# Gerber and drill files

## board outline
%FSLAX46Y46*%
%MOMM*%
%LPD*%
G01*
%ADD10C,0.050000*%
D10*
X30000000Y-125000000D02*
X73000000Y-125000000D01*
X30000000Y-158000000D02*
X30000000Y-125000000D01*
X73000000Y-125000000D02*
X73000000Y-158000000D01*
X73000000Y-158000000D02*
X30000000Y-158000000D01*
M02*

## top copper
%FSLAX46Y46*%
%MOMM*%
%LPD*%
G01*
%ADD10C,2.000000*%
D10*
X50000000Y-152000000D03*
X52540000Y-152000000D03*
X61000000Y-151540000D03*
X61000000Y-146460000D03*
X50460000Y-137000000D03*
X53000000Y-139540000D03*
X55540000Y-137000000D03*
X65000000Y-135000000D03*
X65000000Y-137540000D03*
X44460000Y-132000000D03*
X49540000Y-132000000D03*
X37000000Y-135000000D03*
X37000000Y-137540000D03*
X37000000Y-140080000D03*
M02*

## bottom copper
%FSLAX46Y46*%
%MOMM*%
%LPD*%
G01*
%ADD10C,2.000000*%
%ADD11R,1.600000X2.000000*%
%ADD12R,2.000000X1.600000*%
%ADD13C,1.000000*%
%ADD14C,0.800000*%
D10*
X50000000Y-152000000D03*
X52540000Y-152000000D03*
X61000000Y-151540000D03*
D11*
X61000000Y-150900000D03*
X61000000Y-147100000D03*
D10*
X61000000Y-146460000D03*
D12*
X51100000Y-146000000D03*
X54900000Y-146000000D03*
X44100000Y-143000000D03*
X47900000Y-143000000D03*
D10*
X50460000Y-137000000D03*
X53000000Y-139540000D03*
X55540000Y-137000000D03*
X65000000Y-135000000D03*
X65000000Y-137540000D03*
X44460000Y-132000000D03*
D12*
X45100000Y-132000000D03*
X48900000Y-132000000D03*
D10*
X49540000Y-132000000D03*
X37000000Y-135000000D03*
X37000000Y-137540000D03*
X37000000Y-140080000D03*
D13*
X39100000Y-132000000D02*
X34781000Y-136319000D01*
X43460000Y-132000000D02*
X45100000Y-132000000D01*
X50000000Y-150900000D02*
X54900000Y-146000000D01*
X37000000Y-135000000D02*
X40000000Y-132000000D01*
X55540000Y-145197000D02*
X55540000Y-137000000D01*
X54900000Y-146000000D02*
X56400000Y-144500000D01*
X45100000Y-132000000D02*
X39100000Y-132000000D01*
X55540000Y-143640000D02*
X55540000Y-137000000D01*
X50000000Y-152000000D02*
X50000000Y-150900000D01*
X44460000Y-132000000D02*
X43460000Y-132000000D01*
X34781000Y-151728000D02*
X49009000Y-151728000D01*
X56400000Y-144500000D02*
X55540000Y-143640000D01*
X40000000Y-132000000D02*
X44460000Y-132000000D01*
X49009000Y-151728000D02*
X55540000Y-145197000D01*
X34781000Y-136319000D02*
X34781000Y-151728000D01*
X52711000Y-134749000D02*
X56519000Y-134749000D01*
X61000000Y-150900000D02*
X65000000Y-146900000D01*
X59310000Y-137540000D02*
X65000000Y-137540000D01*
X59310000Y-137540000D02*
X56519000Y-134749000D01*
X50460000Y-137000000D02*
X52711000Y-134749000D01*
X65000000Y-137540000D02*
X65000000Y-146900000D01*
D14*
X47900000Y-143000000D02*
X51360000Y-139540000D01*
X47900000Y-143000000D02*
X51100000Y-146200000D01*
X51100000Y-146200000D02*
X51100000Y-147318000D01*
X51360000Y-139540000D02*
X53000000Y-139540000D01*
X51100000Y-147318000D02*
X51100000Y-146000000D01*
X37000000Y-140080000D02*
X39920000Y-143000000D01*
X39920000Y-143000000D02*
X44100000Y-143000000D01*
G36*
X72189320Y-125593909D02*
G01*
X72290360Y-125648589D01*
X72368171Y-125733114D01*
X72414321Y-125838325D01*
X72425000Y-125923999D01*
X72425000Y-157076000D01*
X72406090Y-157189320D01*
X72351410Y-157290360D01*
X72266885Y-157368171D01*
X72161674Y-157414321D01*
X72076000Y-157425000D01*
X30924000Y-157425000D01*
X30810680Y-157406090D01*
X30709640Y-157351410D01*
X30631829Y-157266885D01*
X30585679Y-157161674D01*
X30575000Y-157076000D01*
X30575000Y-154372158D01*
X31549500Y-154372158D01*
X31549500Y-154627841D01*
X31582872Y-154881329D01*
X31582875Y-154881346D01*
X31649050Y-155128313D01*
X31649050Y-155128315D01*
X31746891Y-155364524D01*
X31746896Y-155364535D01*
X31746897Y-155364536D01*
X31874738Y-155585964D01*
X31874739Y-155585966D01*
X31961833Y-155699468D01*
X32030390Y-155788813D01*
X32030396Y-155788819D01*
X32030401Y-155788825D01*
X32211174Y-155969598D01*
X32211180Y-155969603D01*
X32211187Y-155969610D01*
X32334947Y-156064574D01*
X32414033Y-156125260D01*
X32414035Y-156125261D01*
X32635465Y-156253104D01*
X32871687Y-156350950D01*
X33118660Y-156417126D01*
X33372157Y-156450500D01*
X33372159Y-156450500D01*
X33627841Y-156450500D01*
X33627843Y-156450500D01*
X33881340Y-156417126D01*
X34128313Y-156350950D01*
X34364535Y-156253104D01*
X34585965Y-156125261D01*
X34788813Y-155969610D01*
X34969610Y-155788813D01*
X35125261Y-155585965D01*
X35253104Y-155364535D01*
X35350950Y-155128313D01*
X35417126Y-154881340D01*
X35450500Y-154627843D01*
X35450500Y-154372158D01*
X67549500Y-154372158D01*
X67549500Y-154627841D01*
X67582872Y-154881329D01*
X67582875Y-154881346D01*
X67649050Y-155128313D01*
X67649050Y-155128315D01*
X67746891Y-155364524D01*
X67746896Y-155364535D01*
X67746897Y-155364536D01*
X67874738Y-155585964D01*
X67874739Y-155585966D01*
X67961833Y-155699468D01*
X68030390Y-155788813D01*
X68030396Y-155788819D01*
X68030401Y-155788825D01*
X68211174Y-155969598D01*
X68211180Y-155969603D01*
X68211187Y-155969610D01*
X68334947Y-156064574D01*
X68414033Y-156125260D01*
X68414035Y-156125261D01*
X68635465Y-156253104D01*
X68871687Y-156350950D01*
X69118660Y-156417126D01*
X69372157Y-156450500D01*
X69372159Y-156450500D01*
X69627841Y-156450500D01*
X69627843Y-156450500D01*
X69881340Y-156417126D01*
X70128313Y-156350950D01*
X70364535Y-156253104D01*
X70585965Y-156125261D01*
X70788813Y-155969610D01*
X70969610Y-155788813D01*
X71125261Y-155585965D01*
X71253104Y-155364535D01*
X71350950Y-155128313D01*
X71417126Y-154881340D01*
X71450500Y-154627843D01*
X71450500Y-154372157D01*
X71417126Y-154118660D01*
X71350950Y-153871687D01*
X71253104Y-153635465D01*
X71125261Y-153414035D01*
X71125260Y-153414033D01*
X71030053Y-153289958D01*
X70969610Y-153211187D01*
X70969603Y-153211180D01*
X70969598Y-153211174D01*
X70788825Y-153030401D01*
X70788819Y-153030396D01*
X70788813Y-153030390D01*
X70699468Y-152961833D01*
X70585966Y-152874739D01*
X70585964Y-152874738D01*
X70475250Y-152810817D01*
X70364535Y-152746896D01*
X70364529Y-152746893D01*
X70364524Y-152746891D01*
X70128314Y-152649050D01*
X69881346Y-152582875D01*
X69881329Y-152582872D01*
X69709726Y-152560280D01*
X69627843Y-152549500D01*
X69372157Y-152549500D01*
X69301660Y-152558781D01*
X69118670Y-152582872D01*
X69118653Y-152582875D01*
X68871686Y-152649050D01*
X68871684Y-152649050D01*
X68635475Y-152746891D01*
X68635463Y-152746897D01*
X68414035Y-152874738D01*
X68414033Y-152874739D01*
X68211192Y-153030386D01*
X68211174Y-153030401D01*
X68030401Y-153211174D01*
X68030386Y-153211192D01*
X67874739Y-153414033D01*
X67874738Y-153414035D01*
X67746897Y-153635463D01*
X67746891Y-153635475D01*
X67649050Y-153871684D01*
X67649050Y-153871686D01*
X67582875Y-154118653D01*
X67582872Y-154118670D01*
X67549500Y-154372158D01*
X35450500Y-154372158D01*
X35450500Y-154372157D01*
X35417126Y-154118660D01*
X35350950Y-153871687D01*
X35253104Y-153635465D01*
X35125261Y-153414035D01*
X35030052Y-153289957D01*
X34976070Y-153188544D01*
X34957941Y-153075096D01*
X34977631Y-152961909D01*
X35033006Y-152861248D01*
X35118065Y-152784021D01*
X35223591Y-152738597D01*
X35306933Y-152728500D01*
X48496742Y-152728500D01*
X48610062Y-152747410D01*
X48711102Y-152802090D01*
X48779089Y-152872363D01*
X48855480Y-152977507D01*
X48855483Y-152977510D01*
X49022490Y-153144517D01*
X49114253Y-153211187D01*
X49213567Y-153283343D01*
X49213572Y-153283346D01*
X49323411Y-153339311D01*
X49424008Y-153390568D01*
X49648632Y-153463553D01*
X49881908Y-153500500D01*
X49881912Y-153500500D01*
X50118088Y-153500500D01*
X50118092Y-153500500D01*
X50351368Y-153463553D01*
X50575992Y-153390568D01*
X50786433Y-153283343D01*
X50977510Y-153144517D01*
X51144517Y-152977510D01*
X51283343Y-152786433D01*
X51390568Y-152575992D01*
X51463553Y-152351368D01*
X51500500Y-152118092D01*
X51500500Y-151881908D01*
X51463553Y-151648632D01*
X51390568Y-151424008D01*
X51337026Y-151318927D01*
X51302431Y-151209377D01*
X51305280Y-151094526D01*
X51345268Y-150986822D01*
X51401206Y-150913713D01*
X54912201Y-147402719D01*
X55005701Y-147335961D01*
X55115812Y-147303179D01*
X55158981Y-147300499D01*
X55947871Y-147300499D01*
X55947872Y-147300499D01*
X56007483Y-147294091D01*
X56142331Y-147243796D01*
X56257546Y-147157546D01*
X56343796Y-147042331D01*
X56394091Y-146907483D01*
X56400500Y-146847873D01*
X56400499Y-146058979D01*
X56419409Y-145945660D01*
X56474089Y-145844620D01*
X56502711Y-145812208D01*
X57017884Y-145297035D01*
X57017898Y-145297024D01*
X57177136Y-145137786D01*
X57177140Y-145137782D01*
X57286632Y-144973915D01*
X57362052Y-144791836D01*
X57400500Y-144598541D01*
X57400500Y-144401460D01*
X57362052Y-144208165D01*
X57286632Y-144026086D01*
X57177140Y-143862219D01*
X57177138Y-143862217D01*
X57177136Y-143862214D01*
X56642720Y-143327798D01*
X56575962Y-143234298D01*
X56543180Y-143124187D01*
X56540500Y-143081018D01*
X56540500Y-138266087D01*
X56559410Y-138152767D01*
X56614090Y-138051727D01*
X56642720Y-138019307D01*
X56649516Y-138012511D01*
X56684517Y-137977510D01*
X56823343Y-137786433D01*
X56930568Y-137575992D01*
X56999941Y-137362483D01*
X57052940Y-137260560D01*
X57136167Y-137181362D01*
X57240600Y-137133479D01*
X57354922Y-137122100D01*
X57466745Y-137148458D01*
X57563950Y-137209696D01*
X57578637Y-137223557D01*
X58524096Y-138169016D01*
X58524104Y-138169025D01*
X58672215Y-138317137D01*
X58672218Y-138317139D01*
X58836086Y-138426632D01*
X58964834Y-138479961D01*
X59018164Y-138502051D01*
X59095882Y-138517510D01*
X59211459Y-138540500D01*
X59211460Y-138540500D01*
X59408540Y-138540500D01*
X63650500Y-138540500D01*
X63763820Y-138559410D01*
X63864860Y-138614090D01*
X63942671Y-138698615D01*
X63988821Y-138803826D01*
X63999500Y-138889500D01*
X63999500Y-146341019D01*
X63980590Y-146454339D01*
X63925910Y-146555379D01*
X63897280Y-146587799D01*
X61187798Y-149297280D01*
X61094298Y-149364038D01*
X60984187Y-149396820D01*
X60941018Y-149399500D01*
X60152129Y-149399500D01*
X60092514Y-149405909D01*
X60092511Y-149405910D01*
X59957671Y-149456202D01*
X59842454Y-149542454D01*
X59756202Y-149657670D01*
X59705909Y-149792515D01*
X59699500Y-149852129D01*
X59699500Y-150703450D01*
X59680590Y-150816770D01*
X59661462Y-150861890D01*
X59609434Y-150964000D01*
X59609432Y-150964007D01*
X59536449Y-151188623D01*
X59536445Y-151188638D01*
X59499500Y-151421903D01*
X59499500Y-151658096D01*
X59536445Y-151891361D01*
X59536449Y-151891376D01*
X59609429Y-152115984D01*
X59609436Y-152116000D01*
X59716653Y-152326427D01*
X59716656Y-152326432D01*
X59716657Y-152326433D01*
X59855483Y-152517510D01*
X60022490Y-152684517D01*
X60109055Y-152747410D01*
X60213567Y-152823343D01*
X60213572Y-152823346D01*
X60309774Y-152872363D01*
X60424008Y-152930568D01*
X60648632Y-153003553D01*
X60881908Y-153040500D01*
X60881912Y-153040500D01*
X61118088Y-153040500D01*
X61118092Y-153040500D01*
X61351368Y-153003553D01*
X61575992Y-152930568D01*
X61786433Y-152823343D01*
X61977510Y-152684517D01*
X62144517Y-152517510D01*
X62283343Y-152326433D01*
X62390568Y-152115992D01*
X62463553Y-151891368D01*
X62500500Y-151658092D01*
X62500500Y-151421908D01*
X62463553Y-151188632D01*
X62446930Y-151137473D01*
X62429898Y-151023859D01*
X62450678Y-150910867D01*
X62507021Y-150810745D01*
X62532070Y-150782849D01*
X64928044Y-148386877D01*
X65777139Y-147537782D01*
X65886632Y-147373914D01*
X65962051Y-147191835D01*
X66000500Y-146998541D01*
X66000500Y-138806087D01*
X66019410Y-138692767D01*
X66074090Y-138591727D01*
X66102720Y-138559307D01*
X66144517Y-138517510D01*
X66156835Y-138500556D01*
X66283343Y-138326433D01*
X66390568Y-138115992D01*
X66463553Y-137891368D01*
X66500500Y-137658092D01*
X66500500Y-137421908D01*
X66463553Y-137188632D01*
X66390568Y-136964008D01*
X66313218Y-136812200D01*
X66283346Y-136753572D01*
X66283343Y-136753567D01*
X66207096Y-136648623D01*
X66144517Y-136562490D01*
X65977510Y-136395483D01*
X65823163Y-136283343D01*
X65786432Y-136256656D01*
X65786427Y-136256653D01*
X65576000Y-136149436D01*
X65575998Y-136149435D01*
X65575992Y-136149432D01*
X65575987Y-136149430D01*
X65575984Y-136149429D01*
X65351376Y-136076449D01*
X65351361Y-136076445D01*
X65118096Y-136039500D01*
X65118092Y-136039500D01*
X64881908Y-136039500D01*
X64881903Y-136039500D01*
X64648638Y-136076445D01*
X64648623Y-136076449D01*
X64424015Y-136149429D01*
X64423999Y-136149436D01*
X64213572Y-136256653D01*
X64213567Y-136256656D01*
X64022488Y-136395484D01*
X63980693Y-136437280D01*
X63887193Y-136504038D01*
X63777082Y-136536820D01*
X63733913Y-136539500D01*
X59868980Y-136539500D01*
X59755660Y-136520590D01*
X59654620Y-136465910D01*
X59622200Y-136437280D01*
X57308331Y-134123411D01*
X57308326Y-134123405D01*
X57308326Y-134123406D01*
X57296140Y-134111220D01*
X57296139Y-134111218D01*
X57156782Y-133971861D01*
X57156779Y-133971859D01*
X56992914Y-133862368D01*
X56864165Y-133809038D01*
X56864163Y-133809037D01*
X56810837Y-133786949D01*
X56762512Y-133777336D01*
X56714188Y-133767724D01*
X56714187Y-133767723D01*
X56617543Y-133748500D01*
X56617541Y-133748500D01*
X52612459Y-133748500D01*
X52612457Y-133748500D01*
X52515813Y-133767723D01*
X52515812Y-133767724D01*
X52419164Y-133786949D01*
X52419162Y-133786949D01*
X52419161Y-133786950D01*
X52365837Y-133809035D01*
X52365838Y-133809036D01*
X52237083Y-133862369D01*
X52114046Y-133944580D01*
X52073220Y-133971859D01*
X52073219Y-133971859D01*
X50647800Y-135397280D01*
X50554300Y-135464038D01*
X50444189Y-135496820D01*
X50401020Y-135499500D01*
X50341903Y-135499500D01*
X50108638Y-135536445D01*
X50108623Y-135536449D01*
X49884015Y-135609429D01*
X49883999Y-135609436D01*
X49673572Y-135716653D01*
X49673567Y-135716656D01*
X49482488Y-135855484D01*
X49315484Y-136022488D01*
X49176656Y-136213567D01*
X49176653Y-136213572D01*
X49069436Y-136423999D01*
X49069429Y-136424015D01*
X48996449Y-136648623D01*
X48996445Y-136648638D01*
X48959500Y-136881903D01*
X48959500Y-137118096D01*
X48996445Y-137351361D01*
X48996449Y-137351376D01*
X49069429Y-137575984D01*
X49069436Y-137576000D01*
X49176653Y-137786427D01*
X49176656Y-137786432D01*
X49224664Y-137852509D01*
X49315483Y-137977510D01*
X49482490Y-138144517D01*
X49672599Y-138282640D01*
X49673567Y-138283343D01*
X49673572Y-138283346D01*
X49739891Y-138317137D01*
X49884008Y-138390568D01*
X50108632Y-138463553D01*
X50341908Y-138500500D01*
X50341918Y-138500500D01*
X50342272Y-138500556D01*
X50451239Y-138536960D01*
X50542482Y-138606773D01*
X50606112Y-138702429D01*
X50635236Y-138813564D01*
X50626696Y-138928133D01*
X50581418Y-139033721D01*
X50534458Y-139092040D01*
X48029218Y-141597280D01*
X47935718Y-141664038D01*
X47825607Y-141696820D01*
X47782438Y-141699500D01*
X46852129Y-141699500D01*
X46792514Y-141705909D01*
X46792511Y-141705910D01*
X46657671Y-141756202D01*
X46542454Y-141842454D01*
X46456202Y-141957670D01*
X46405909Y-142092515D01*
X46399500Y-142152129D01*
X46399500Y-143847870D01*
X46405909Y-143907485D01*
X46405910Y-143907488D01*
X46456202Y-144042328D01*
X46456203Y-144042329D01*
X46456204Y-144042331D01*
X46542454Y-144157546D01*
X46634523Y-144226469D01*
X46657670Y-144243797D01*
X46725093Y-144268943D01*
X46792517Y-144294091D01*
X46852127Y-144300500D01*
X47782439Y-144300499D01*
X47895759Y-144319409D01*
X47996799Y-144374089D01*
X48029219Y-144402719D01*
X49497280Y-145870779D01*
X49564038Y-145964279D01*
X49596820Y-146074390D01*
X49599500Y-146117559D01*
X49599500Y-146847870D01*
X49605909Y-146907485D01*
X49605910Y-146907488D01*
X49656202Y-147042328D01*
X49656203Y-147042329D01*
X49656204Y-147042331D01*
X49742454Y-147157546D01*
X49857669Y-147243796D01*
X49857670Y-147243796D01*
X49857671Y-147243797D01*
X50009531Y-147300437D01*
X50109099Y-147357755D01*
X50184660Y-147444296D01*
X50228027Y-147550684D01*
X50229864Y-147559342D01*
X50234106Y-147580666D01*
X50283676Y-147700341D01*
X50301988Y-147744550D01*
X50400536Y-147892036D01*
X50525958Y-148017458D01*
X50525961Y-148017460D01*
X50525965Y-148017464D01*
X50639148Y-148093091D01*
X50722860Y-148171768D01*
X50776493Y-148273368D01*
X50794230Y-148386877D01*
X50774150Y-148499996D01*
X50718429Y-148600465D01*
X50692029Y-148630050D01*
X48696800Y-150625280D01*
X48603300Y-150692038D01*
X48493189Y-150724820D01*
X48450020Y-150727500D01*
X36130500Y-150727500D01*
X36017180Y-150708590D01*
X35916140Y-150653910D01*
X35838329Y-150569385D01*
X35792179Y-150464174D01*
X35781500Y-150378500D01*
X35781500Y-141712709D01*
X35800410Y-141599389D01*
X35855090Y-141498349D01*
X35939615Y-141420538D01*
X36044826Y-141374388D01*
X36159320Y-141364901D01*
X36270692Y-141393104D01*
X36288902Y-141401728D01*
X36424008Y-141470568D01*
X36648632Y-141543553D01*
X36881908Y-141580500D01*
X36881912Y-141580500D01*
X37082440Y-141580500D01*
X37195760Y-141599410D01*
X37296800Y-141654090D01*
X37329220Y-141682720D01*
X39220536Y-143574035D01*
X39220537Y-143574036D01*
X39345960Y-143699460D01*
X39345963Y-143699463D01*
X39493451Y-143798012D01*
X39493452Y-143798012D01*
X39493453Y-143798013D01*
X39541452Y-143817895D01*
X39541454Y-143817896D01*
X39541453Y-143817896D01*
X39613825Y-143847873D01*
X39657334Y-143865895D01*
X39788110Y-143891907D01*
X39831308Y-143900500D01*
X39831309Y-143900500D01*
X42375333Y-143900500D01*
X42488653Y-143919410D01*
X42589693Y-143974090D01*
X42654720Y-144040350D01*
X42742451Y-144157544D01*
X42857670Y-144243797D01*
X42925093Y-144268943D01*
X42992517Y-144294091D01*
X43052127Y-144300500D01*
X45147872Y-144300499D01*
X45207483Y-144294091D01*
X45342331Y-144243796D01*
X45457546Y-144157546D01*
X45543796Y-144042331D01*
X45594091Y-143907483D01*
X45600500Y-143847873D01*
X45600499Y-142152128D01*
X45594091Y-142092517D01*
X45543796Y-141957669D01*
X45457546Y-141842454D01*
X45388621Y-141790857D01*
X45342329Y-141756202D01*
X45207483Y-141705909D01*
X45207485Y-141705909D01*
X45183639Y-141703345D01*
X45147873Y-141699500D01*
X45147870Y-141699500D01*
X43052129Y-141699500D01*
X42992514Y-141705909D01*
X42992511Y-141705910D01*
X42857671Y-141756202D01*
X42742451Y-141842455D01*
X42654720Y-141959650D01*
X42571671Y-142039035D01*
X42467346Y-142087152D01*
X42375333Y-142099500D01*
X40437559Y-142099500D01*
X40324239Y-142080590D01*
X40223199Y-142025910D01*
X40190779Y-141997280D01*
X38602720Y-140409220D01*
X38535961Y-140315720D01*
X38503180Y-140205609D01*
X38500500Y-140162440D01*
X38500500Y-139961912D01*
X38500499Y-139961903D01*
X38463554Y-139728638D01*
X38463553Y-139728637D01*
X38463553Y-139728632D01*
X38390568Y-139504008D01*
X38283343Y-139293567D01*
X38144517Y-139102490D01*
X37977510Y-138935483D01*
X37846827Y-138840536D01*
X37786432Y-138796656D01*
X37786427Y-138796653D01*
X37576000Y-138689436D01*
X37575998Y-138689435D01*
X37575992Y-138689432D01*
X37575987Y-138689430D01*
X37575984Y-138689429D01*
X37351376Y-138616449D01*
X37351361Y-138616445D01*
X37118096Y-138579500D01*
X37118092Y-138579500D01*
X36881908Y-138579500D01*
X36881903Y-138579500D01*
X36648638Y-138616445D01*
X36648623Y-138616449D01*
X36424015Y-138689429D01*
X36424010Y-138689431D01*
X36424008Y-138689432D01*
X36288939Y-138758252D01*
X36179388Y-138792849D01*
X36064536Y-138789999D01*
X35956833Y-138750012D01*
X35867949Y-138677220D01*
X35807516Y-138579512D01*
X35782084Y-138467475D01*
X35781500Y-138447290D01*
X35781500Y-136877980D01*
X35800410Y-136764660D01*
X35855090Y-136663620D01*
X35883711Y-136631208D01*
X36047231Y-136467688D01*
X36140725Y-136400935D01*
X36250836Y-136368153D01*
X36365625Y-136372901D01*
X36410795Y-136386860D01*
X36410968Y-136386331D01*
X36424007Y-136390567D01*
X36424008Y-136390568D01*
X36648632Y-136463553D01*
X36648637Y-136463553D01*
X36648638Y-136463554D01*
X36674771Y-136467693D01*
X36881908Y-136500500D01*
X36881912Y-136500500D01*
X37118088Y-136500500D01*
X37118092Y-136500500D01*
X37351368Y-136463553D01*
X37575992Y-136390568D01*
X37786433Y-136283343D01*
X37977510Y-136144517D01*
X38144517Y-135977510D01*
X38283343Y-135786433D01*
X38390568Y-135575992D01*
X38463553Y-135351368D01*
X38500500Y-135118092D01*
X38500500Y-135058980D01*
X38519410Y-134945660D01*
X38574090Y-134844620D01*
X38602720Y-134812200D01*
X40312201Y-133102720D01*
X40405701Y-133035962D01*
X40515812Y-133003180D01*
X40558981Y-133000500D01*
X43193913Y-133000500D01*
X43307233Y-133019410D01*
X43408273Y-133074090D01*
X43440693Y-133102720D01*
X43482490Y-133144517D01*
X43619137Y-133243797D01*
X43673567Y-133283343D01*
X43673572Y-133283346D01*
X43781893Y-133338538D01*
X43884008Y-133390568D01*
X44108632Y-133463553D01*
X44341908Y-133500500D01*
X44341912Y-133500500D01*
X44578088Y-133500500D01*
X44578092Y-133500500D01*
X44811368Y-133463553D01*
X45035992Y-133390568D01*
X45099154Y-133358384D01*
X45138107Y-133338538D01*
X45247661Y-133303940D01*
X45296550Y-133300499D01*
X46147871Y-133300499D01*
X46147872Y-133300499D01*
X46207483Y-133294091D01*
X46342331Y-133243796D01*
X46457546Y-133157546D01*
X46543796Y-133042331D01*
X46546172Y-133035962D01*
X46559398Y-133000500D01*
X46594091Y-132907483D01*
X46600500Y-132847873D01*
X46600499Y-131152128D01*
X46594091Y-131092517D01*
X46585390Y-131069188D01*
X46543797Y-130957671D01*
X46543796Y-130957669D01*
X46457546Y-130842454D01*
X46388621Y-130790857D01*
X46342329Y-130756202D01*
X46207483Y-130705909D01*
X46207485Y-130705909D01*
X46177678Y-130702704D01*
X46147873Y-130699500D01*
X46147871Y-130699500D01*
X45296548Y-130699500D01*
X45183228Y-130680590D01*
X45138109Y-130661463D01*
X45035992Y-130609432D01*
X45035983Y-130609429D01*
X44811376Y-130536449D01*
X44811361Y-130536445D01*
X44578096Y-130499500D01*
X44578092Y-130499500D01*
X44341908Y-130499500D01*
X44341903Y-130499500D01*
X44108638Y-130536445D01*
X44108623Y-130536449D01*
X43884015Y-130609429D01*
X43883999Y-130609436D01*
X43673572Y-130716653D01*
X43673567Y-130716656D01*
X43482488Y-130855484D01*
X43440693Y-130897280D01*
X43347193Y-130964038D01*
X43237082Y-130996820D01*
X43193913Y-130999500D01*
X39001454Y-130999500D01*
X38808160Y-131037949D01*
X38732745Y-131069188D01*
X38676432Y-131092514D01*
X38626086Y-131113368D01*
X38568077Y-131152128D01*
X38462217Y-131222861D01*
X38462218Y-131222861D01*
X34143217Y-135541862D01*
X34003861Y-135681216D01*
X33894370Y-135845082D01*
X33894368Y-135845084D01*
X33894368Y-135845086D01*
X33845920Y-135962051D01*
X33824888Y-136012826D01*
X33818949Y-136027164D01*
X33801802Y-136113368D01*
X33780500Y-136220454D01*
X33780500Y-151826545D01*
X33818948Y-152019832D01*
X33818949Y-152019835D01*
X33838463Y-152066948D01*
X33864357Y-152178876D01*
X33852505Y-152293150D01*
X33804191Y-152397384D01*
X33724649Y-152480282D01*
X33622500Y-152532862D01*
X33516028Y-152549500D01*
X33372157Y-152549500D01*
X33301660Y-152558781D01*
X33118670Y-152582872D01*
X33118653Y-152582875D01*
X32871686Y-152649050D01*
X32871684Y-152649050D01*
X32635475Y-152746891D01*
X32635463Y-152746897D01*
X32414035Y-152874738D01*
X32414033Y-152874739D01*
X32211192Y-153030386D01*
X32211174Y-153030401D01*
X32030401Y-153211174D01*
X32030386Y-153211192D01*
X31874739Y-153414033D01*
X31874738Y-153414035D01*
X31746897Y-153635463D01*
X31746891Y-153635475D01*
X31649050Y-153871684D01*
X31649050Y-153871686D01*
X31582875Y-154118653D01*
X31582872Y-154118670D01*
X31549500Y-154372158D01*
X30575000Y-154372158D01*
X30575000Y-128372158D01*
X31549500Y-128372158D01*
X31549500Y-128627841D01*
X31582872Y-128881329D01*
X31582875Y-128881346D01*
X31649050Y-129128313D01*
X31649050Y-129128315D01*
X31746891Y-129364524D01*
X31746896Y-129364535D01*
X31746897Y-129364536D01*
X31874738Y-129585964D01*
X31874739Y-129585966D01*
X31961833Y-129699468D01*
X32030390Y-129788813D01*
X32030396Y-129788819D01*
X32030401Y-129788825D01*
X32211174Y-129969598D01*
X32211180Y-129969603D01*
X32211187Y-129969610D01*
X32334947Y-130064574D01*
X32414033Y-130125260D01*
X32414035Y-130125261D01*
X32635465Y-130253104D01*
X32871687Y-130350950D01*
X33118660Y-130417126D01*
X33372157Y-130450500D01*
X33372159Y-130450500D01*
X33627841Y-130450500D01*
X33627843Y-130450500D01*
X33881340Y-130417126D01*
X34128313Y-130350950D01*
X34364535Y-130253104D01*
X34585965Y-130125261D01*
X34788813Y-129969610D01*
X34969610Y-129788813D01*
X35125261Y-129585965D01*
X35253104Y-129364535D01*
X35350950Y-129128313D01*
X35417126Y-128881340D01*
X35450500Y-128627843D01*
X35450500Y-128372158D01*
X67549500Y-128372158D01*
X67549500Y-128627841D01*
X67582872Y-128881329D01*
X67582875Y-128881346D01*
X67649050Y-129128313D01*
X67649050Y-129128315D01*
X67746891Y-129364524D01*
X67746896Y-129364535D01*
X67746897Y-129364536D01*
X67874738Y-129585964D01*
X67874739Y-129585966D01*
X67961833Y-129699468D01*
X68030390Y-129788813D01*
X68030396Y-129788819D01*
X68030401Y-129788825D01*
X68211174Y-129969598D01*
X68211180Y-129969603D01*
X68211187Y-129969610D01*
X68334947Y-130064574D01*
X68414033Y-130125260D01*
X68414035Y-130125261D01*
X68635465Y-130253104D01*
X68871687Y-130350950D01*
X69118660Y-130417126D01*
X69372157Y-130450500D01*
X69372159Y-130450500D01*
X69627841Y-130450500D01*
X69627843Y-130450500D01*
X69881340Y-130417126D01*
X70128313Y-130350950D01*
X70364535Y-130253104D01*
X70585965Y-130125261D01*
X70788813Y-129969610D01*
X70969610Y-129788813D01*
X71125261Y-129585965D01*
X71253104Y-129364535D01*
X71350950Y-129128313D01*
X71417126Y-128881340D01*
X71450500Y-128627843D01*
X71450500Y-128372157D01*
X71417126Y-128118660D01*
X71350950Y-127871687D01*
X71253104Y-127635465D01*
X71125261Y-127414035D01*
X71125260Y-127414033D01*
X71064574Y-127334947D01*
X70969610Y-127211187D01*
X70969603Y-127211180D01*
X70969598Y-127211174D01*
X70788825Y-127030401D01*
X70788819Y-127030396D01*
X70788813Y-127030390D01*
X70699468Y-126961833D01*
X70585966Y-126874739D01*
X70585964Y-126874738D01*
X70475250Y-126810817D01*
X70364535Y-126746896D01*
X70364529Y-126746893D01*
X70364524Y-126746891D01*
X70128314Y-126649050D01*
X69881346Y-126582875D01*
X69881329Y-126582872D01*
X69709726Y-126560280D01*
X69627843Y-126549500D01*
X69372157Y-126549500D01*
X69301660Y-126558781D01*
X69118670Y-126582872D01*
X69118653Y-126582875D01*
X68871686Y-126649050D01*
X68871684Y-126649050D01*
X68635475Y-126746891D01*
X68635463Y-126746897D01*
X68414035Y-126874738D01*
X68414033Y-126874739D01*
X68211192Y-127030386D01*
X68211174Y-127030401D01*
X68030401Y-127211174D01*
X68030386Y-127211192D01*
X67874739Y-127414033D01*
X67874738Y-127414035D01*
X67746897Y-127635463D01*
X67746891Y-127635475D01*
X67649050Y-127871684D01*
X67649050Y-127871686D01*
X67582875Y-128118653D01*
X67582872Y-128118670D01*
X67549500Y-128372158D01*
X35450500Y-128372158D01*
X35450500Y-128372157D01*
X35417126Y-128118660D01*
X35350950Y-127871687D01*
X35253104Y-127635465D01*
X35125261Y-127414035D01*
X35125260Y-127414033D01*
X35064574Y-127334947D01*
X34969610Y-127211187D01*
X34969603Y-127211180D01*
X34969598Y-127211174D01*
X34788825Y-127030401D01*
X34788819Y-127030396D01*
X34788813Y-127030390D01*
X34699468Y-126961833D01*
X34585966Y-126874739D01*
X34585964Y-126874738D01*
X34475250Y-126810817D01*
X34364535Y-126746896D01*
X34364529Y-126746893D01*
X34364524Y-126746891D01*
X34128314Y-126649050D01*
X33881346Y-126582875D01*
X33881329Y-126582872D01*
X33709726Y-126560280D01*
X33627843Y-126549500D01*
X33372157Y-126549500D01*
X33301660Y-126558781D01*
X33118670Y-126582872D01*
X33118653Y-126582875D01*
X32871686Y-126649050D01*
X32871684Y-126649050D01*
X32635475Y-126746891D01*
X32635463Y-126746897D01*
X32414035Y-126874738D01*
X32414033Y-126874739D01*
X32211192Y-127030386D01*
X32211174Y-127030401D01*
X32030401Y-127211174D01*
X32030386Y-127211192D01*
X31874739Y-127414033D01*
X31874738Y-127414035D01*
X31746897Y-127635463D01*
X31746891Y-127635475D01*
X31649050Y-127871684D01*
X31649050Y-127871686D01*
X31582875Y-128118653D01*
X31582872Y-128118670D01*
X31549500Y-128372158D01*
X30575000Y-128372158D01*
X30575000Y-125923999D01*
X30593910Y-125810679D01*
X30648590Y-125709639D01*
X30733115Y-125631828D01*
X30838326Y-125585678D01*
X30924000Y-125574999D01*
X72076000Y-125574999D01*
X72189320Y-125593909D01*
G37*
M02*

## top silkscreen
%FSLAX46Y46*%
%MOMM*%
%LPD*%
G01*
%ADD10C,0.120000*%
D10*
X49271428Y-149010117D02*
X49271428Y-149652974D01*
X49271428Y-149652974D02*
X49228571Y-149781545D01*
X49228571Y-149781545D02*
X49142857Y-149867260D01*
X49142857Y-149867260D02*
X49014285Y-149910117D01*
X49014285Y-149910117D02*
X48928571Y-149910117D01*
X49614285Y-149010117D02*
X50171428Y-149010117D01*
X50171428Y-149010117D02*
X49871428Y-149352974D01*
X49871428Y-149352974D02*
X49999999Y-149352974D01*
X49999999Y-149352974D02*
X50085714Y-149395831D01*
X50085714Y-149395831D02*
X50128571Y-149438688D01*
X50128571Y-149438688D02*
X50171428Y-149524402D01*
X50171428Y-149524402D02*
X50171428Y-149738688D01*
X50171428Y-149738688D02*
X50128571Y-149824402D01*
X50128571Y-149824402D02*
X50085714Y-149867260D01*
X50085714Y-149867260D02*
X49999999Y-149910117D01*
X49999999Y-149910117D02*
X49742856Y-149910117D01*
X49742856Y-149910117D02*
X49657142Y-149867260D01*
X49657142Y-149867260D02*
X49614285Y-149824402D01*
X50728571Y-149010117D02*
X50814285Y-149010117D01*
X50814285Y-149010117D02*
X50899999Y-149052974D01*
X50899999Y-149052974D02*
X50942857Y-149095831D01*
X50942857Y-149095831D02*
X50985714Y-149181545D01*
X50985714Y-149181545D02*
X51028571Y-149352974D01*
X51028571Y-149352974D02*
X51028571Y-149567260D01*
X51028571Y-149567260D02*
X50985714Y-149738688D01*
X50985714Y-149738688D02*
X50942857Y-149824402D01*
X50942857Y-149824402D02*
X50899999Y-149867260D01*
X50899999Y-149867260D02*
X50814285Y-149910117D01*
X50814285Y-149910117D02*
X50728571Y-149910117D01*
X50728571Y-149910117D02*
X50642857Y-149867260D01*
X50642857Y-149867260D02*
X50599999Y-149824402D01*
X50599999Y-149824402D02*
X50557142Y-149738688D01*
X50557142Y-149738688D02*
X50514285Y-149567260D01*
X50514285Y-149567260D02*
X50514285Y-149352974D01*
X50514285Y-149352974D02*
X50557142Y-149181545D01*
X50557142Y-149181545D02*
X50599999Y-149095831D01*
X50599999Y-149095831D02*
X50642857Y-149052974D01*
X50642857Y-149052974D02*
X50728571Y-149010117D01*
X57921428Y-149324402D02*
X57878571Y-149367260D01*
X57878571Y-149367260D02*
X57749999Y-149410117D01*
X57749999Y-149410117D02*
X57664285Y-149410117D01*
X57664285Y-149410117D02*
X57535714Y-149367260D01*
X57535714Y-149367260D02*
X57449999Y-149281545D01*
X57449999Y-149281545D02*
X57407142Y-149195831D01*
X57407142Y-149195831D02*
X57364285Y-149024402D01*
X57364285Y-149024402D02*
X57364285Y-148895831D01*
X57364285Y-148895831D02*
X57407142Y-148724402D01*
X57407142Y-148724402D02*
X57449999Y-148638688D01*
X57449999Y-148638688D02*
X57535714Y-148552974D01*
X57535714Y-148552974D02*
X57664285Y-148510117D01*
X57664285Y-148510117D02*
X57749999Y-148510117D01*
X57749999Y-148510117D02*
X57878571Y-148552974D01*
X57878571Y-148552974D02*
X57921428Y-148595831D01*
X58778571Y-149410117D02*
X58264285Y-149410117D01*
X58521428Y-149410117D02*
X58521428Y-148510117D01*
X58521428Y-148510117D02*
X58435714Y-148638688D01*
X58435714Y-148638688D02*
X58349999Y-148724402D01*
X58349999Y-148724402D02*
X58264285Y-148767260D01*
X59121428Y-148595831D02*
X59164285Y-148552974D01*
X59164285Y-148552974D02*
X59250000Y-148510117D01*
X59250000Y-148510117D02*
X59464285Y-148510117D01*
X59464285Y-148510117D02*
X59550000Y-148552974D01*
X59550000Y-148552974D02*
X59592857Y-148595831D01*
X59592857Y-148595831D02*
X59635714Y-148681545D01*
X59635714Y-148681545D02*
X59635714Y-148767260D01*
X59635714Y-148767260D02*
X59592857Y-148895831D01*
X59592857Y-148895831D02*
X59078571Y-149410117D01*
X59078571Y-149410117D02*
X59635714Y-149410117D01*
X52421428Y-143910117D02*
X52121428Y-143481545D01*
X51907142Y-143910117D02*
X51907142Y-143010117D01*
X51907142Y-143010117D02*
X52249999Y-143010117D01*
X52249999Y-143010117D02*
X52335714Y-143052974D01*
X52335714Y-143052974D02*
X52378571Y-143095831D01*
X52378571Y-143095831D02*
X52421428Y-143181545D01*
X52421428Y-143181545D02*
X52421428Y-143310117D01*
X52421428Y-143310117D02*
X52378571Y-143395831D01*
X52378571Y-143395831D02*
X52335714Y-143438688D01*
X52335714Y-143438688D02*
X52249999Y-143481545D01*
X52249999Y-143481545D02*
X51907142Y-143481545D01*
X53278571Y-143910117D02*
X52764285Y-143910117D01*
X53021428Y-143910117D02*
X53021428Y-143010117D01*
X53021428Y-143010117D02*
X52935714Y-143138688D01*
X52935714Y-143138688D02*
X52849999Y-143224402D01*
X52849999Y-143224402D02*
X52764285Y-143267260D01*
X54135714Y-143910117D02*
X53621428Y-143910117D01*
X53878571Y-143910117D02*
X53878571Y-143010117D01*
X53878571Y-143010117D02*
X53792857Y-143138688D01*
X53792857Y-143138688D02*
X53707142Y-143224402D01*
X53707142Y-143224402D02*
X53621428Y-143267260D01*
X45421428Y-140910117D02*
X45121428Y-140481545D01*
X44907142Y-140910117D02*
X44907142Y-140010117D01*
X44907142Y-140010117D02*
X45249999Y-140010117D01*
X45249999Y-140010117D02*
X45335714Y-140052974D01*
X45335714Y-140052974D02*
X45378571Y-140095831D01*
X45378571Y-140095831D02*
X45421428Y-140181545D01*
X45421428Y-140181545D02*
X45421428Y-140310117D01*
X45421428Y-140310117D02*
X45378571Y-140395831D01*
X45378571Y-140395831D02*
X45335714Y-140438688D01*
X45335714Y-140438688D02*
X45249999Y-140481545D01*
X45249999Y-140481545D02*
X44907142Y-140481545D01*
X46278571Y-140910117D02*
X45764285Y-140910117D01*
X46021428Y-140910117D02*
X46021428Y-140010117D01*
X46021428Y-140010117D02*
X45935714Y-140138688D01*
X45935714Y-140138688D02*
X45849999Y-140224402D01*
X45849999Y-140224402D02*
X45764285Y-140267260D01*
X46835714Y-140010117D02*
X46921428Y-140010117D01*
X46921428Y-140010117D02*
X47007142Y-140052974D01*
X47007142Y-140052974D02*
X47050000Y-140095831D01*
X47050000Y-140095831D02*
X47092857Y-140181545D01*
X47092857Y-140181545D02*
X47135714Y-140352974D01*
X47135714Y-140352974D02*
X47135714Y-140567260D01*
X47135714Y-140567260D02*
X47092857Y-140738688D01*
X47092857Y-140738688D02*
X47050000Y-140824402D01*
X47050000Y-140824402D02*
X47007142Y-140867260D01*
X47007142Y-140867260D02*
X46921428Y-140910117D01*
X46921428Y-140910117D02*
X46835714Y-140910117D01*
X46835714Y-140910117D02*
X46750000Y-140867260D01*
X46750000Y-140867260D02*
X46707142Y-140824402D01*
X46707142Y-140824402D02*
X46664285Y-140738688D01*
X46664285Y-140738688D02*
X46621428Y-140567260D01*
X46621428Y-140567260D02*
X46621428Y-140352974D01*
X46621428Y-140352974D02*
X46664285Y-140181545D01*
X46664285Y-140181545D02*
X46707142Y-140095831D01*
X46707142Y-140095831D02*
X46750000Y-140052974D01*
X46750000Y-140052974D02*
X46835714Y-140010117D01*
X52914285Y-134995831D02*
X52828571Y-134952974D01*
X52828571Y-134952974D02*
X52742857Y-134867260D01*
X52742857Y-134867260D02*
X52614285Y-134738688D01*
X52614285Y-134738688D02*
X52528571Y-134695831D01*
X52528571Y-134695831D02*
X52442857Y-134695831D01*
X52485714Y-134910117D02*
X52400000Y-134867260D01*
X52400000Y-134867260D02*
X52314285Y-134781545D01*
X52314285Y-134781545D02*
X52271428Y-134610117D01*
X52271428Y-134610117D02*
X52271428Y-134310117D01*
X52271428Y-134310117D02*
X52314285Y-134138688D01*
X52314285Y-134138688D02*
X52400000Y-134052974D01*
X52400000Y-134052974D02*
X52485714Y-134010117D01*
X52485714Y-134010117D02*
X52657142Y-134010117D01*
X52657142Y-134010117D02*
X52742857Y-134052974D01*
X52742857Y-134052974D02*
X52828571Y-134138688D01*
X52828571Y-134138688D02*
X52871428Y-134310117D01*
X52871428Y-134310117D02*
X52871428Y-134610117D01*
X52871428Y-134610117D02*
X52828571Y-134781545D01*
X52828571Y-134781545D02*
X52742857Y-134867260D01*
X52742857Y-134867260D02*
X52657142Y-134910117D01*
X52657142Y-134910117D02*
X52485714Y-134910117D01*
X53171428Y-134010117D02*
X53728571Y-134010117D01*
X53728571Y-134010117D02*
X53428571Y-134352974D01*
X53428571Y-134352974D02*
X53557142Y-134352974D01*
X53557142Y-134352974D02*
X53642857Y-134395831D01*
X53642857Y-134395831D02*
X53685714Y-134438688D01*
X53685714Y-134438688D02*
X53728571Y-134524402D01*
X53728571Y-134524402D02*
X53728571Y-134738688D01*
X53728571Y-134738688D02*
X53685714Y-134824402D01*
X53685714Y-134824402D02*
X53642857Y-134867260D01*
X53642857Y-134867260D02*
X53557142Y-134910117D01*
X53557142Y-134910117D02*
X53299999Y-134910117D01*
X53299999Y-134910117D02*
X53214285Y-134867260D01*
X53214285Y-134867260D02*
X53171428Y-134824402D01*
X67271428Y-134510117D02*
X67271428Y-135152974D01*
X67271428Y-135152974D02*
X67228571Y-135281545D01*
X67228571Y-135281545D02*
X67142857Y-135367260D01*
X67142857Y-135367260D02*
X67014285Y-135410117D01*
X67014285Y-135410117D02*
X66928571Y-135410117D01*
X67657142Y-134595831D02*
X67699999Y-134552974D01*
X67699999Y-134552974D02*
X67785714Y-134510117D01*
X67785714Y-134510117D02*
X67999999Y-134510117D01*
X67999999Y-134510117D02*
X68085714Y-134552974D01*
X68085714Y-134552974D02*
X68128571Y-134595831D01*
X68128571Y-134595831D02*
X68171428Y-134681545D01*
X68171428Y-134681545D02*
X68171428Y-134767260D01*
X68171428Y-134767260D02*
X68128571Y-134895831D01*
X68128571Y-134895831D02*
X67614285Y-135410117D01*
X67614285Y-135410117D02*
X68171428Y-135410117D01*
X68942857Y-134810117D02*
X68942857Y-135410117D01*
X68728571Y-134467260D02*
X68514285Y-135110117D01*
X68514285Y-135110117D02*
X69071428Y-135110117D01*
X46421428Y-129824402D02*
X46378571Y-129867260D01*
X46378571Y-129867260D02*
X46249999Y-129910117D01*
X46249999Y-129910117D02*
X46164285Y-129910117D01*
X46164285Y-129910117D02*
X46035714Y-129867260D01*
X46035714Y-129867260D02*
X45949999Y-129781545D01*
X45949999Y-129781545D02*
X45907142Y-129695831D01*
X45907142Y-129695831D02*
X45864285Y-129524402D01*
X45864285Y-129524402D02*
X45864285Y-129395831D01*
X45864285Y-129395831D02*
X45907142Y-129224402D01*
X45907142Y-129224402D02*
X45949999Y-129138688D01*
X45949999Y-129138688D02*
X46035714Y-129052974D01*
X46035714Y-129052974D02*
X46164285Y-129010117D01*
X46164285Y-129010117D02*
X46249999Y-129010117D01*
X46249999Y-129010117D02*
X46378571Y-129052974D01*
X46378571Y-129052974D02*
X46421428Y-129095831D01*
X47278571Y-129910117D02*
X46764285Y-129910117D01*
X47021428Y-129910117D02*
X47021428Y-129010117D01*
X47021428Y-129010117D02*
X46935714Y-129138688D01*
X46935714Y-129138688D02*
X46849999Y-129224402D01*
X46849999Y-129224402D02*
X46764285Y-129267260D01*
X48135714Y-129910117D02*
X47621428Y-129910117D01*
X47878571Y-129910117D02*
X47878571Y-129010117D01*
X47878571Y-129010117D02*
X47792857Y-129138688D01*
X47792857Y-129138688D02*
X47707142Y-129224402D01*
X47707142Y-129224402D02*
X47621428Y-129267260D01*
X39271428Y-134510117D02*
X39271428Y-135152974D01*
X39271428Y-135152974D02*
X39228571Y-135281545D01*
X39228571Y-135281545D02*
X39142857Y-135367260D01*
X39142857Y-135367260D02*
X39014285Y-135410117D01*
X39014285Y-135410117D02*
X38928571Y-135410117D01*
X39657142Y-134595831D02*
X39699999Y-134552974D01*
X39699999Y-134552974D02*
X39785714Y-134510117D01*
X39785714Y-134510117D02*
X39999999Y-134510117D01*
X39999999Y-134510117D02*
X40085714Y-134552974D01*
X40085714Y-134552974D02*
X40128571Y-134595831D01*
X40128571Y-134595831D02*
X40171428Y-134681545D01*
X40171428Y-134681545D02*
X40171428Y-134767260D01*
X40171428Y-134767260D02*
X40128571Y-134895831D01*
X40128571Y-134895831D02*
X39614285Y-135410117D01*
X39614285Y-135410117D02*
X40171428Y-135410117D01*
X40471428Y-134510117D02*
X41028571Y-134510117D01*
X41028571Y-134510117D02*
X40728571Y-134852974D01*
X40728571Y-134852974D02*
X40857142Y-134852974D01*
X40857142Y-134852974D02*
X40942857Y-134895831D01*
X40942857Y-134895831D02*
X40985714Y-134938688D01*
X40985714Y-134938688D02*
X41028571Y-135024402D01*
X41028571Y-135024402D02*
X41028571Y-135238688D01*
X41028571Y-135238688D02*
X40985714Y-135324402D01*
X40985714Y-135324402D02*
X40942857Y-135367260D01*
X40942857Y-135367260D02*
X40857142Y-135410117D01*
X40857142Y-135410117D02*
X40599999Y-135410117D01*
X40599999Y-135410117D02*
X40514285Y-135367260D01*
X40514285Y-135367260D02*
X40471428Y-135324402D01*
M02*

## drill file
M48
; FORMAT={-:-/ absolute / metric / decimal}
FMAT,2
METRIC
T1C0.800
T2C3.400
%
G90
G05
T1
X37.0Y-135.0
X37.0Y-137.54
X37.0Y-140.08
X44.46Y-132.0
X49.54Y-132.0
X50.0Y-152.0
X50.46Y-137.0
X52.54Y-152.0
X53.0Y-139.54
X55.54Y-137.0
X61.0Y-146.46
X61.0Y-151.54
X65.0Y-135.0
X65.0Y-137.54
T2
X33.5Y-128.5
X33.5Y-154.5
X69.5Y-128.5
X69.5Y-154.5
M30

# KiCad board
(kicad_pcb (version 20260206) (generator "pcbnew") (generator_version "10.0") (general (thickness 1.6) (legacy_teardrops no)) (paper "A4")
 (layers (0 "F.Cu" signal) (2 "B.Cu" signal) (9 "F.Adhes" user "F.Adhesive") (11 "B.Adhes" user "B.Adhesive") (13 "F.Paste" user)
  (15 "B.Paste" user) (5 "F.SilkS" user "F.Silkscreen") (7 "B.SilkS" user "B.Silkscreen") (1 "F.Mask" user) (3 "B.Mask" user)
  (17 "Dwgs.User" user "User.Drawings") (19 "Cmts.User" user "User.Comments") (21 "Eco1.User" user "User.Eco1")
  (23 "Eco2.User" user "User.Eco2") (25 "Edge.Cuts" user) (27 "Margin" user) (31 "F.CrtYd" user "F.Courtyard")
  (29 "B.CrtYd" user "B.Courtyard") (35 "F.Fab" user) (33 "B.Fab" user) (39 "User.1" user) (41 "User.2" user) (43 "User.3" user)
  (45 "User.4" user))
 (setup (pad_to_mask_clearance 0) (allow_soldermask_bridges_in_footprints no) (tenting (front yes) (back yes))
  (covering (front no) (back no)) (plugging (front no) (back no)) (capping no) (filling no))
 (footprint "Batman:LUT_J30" (layer "F.Cu") (at 50 152)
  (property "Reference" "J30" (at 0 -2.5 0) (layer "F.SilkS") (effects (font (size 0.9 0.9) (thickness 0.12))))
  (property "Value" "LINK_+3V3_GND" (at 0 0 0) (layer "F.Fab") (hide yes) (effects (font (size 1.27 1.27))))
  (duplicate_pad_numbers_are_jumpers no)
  (pad "1" thru_hole circle (at 0 0) (size 2 2) (drill 0.8) (layers "*.Cu") (remove_unused_layers no) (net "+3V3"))
  (pad "2" thru_hole circle (at 2.54 0) (size 2 2) (drill 0.8) (layers "*.Cu") (remove_unused_layers no) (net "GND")))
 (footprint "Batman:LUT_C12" (layer "F.Cu") (at 61 149 90)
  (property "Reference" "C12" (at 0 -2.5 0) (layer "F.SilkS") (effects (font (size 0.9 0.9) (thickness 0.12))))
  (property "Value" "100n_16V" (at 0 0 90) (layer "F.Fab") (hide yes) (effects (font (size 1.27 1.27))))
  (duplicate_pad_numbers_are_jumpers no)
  (pad "1" thru_hole circle (at -2.54 0 90) (size 2 2) (drill 0.8) (layers "*.Cu") (remove_unused_layers no) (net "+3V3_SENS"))
  (pad "1" smd rect (at -1.9 0 90) (size 2 1.6) (layers "B.Cu") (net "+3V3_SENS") (thermal_bridge_angle 45))
  (pad "2" smd rect (at 1.9 0 90) (size 2 1.6) (layers "B.Cu") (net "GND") (thermal_bridge_angle 45))
  (pad "2" thru_hole circle (at 2.54 0 90) (size 2 2) (drill 0.8) (layers "*.Cu") (remove_unused_layers no) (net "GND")))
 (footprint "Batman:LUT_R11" (layer "F.Cu") (at 53 146)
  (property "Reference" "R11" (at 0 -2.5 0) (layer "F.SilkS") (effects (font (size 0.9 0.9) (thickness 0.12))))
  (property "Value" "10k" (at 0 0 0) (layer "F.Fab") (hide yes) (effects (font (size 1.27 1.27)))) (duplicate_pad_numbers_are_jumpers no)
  (pad "1" smd rect (at -1.9 0) (size 2 1.6) (layers "B.Cu") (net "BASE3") (thermal_bridge_angle 45))
  (pad "2" smd rect (at 1.9 0) (size 2 1.6) (layers "B.Cu") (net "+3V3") (thermal_bridge_angle 45)))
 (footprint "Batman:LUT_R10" (layer "F.Cu") (at 46 143)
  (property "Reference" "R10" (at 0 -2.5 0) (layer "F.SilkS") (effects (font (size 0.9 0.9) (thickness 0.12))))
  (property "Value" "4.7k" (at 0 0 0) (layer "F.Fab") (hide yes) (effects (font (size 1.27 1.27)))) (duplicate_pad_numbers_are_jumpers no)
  (pad "1" smd rect (at -1.9 0) (size 2 1.6) (layers "B.Cu") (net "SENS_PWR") (thermal_bridge_angle 45))
  (pad "2" smd rect (at 1.9 0) (size 2 1.6) (layers "B.Cu") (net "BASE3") (thermal_bridge_angle 45)))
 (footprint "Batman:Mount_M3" (layer "F.Cu") (at 69.5 128.5)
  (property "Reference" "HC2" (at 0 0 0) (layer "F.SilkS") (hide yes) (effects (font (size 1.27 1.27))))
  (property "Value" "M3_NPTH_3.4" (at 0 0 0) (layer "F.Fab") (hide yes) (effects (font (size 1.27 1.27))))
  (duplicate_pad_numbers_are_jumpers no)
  (pad "" np_thru_hole circle (at 0 0) (size 3.4 3.4) (drill 3.4) (layers "*.Cu")))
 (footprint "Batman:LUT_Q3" (layer "F.Cu") (at 53 137)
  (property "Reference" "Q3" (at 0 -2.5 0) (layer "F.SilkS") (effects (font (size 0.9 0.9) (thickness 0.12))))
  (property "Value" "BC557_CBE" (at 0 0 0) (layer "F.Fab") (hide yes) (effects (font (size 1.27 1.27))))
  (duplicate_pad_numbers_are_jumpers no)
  (pad "1" thru_hole circle (at -2.54 0) (size 2 2) (drill 0.8) (layers "*.Cu") (remove_unused_layers no) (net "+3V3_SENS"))
  (pad "2" thru_hole circle (at 0 2.54) (size 2 2) (drill 0.8) (layers "*.Cu") (remove_unused_layers no) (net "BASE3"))
  (pad "3" thru_hole circle (at 2.54 0) (size 2 2) (drill 0.8) (layers "*.Cu") (remove_unused_layers no) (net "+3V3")))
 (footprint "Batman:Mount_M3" (layer "F.Cu") (at 69.5 154.5)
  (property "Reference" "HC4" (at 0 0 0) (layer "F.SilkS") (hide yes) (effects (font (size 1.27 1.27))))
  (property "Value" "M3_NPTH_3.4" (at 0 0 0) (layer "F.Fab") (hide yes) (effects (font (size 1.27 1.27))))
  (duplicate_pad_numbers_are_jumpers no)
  (pad "" np_thru_hole circle (at 0 0) (size 3.4 3.4) (drill 3.4) (layers "*.Cu")))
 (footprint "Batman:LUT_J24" (layer "F.Cu") (at 65 135 -90)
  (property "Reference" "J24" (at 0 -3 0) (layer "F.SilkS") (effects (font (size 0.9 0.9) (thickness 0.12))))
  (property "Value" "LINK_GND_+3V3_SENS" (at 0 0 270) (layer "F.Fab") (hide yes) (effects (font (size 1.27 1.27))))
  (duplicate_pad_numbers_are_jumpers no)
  (pad "1" thru_hole circle (at 0 0 270) (size 2 2) (drill 0.8) (layers "*.Cu") (remove_unused_layers no) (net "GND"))
  (pad "2" thru_hole circle (at 2.54 0 270) (size 2 2) (drill 0.8) (layers "*.Cu") (remove_unused_layers no) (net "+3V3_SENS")))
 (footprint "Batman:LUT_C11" (layer "F.Cu") (at 47 132)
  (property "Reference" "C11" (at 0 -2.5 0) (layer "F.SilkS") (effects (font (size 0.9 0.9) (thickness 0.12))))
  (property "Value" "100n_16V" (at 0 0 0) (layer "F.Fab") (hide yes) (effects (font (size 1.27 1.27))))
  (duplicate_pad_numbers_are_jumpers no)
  (pad "1" thru_hole circle (at -2.54 0) (size 2 2) (drill 0.8) (layers "*.Cu") (remove_unused_layers no) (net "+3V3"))
  (pad "1" smd rect (at -1.9 0) (size 2 1.6) (layers "B.Cu") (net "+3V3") (thermal_bridge_angle 45))
  (pad "2" smd rect (at 1.9 0) (size 2 1.6) (layers "B.Cu") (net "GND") (thermal_bridge_angle 45))
  (pad "2" thru_hole circle (at 2.54 0) (size 2 2) (drill 0.8) (layers "*.Cu") (remove_unused_layers no) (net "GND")))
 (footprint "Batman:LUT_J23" (layer "F.Cu") (at 37 135 -90)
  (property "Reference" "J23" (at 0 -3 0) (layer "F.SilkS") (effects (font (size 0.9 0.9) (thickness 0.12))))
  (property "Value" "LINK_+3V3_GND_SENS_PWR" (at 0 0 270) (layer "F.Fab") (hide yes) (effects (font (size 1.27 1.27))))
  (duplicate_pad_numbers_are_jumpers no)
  (pad "1" thru_hole circle (at 0 0 270) (size 2 2) (drill 0.8) (layers "*.Cu") (remove_unused_layers no) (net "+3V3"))
  (pad "2" thru_hole circle (at 2.54 0 270) (size 2 2) (drill 0.8) (layers "*.Cu") (remove_unused_layers no) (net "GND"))
  (pad "3" thru_hole circle (at 5.08 0 270) (size 2 2) (drill 0.8) (layers "*.Cu") (remove_unused_layers no) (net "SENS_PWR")))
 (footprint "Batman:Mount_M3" (layer "F.Cu") (at 33.5 128.5)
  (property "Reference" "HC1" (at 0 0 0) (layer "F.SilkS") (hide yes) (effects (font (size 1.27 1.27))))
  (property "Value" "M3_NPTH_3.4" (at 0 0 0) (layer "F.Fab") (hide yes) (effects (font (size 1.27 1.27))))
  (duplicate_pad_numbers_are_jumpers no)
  (pad "" np_thru_hole circle (at 0 0) (size 3.4 3.4) (drill 3.4) (layers "*.Cu")))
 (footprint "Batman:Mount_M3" (layer "F.Cu") (at 33.5 154.5)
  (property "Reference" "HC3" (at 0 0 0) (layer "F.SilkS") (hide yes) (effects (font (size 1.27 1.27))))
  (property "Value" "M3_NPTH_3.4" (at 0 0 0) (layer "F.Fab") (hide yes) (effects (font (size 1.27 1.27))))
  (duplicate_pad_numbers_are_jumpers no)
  (pad "" np_thru_hole circle (at 0 0) (size 3.4 3.4) (drill 3.4) (layers "*.Cu")))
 (gr_line (start 30 125) (end 73 125) (stroke (width 0.05) (type default)) (layer "Edge.Cuts"))
 (gr_line (start 30 158) (end 30 125) (stroke (width 0.05) (type default)) (layer "Edge.Cuts"))
 (gr_line (start 73 125) (end 73 158) (stroke (width 0.05) (type default)) (layer "Edge.Cuts"))
 (gr_line (start 73 158) (end 30 158) (stroke (width 0.05) (type default)) (layer "Edge.Cuts"))
 (segment (start 39.1 132) (end 34.781 136.319) (width 1) (layer "B.Cu") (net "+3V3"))
 (segment (start 43.46 132) (end 45.1 132) (width 1) (layer "B.Cu") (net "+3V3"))
 (segment (start 50 150.9) (end 54.9 146) (width 1) (layer "B.Cu") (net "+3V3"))
 (segment (start 37 135) (end 40 132) (width 1) (layer "B.Cu") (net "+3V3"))
 (segment (start 55.54 145.197) (end 55.54 137) (width 1) (layer "B.Cu") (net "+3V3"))
 (segment (start 54.9 146) (end 56.4 144.5) (width 1) (layer "B.Cu") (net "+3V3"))
 (segment (start 45.1 132) (end 39.1 132) (width 1) (layer "B.Cu") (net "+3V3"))
 (segment (start 55.54 143.64) (end 55.54 137) (width 1) (layer "B.Cu") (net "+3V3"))
 (segment (start 50 152) (end 50 150.9) (width 1) (layer "B.Cu") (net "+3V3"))
 (segment (start 44.46 132) (end 43.46 132) (width 1) (layer "B.Cu") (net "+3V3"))
 (segment (start 34.781 151.728) (end 49.009 151.728) (width 1) (layer "B.Cu") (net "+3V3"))
 (segment (start 56.4 144.5) (end 55.54 143.64) (width 1) (layer "B.Cu") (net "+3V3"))
 (segment (start 40 132) (end 44.46 132) (width 1) (layer "B.Cu") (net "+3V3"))
 (segment (start 49.009 151.728) (end 55.54 145.197) (width 1) (layer "B.Cu") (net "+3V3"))
 (segment (start 34.781 136.319) (end 34.781 151.728) (width 1) (layer "B.Cu") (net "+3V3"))
 (segment (start 52.711 134.749) (end 56.519 134.749) (width 1) (layer "B.Cu") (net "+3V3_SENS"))
 (segment (start 61 150.9) (end 65 146.9) (width 1) (layer "B.Cu") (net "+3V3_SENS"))
 (segment (start 59.31 137.54) (end 65 137.54) (width 1) (layer "B.Cu") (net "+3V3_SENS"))
 (segment (start 59.31 137.54) (end 56.519 134.749) (width 1) (layer "B.Cu") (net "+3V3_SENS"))
 (segment (start 50.46 137) (end 52.711 134.749) (width 1) (layer "B.Cu") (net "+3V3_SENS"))
 (segment (start 65 137.54) (end 65 146.9) (width 1) (layer "B.Cu") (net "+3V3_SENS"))
 (segment (start 47.9 143) (end 51.36 139.54) (width 0.8) (layer "B.Cu") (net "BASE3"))
 (segment (start 47.9 143) (end 51.1 146.2) (width 0.8) (layer "B.Cu") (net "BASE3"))
 (segment (start 51.1 146.2) (end 51.1 147.318) (width 0.8) (layer "B.Cu") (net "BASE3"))
 (segment (start 51.36 139.54) (end 53 139.54) (width 0.8) (layer "B.Cu") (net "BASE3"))
 (segment (start 51.1 147.318) (end 51.1 146) (width 0.8) (layer "B.Cu") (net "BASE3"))
 (segment (start 37 140.08) (end 39.92 143) (width 0.8) (layer "B.Cu") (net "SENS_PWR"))
 (segment (start 39.92 143) (end 44.1 143) (width 0.8) (layer "B.Cu") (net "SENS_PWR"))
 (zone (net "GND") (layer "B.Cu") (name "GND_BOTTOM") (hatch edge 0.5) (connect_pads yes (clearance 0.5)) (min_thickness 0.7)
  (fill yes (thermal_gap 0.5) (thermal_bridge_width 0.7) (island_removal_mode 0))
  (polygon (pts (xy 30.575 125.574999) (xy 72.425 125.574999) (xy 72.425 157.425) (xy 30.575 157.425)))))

